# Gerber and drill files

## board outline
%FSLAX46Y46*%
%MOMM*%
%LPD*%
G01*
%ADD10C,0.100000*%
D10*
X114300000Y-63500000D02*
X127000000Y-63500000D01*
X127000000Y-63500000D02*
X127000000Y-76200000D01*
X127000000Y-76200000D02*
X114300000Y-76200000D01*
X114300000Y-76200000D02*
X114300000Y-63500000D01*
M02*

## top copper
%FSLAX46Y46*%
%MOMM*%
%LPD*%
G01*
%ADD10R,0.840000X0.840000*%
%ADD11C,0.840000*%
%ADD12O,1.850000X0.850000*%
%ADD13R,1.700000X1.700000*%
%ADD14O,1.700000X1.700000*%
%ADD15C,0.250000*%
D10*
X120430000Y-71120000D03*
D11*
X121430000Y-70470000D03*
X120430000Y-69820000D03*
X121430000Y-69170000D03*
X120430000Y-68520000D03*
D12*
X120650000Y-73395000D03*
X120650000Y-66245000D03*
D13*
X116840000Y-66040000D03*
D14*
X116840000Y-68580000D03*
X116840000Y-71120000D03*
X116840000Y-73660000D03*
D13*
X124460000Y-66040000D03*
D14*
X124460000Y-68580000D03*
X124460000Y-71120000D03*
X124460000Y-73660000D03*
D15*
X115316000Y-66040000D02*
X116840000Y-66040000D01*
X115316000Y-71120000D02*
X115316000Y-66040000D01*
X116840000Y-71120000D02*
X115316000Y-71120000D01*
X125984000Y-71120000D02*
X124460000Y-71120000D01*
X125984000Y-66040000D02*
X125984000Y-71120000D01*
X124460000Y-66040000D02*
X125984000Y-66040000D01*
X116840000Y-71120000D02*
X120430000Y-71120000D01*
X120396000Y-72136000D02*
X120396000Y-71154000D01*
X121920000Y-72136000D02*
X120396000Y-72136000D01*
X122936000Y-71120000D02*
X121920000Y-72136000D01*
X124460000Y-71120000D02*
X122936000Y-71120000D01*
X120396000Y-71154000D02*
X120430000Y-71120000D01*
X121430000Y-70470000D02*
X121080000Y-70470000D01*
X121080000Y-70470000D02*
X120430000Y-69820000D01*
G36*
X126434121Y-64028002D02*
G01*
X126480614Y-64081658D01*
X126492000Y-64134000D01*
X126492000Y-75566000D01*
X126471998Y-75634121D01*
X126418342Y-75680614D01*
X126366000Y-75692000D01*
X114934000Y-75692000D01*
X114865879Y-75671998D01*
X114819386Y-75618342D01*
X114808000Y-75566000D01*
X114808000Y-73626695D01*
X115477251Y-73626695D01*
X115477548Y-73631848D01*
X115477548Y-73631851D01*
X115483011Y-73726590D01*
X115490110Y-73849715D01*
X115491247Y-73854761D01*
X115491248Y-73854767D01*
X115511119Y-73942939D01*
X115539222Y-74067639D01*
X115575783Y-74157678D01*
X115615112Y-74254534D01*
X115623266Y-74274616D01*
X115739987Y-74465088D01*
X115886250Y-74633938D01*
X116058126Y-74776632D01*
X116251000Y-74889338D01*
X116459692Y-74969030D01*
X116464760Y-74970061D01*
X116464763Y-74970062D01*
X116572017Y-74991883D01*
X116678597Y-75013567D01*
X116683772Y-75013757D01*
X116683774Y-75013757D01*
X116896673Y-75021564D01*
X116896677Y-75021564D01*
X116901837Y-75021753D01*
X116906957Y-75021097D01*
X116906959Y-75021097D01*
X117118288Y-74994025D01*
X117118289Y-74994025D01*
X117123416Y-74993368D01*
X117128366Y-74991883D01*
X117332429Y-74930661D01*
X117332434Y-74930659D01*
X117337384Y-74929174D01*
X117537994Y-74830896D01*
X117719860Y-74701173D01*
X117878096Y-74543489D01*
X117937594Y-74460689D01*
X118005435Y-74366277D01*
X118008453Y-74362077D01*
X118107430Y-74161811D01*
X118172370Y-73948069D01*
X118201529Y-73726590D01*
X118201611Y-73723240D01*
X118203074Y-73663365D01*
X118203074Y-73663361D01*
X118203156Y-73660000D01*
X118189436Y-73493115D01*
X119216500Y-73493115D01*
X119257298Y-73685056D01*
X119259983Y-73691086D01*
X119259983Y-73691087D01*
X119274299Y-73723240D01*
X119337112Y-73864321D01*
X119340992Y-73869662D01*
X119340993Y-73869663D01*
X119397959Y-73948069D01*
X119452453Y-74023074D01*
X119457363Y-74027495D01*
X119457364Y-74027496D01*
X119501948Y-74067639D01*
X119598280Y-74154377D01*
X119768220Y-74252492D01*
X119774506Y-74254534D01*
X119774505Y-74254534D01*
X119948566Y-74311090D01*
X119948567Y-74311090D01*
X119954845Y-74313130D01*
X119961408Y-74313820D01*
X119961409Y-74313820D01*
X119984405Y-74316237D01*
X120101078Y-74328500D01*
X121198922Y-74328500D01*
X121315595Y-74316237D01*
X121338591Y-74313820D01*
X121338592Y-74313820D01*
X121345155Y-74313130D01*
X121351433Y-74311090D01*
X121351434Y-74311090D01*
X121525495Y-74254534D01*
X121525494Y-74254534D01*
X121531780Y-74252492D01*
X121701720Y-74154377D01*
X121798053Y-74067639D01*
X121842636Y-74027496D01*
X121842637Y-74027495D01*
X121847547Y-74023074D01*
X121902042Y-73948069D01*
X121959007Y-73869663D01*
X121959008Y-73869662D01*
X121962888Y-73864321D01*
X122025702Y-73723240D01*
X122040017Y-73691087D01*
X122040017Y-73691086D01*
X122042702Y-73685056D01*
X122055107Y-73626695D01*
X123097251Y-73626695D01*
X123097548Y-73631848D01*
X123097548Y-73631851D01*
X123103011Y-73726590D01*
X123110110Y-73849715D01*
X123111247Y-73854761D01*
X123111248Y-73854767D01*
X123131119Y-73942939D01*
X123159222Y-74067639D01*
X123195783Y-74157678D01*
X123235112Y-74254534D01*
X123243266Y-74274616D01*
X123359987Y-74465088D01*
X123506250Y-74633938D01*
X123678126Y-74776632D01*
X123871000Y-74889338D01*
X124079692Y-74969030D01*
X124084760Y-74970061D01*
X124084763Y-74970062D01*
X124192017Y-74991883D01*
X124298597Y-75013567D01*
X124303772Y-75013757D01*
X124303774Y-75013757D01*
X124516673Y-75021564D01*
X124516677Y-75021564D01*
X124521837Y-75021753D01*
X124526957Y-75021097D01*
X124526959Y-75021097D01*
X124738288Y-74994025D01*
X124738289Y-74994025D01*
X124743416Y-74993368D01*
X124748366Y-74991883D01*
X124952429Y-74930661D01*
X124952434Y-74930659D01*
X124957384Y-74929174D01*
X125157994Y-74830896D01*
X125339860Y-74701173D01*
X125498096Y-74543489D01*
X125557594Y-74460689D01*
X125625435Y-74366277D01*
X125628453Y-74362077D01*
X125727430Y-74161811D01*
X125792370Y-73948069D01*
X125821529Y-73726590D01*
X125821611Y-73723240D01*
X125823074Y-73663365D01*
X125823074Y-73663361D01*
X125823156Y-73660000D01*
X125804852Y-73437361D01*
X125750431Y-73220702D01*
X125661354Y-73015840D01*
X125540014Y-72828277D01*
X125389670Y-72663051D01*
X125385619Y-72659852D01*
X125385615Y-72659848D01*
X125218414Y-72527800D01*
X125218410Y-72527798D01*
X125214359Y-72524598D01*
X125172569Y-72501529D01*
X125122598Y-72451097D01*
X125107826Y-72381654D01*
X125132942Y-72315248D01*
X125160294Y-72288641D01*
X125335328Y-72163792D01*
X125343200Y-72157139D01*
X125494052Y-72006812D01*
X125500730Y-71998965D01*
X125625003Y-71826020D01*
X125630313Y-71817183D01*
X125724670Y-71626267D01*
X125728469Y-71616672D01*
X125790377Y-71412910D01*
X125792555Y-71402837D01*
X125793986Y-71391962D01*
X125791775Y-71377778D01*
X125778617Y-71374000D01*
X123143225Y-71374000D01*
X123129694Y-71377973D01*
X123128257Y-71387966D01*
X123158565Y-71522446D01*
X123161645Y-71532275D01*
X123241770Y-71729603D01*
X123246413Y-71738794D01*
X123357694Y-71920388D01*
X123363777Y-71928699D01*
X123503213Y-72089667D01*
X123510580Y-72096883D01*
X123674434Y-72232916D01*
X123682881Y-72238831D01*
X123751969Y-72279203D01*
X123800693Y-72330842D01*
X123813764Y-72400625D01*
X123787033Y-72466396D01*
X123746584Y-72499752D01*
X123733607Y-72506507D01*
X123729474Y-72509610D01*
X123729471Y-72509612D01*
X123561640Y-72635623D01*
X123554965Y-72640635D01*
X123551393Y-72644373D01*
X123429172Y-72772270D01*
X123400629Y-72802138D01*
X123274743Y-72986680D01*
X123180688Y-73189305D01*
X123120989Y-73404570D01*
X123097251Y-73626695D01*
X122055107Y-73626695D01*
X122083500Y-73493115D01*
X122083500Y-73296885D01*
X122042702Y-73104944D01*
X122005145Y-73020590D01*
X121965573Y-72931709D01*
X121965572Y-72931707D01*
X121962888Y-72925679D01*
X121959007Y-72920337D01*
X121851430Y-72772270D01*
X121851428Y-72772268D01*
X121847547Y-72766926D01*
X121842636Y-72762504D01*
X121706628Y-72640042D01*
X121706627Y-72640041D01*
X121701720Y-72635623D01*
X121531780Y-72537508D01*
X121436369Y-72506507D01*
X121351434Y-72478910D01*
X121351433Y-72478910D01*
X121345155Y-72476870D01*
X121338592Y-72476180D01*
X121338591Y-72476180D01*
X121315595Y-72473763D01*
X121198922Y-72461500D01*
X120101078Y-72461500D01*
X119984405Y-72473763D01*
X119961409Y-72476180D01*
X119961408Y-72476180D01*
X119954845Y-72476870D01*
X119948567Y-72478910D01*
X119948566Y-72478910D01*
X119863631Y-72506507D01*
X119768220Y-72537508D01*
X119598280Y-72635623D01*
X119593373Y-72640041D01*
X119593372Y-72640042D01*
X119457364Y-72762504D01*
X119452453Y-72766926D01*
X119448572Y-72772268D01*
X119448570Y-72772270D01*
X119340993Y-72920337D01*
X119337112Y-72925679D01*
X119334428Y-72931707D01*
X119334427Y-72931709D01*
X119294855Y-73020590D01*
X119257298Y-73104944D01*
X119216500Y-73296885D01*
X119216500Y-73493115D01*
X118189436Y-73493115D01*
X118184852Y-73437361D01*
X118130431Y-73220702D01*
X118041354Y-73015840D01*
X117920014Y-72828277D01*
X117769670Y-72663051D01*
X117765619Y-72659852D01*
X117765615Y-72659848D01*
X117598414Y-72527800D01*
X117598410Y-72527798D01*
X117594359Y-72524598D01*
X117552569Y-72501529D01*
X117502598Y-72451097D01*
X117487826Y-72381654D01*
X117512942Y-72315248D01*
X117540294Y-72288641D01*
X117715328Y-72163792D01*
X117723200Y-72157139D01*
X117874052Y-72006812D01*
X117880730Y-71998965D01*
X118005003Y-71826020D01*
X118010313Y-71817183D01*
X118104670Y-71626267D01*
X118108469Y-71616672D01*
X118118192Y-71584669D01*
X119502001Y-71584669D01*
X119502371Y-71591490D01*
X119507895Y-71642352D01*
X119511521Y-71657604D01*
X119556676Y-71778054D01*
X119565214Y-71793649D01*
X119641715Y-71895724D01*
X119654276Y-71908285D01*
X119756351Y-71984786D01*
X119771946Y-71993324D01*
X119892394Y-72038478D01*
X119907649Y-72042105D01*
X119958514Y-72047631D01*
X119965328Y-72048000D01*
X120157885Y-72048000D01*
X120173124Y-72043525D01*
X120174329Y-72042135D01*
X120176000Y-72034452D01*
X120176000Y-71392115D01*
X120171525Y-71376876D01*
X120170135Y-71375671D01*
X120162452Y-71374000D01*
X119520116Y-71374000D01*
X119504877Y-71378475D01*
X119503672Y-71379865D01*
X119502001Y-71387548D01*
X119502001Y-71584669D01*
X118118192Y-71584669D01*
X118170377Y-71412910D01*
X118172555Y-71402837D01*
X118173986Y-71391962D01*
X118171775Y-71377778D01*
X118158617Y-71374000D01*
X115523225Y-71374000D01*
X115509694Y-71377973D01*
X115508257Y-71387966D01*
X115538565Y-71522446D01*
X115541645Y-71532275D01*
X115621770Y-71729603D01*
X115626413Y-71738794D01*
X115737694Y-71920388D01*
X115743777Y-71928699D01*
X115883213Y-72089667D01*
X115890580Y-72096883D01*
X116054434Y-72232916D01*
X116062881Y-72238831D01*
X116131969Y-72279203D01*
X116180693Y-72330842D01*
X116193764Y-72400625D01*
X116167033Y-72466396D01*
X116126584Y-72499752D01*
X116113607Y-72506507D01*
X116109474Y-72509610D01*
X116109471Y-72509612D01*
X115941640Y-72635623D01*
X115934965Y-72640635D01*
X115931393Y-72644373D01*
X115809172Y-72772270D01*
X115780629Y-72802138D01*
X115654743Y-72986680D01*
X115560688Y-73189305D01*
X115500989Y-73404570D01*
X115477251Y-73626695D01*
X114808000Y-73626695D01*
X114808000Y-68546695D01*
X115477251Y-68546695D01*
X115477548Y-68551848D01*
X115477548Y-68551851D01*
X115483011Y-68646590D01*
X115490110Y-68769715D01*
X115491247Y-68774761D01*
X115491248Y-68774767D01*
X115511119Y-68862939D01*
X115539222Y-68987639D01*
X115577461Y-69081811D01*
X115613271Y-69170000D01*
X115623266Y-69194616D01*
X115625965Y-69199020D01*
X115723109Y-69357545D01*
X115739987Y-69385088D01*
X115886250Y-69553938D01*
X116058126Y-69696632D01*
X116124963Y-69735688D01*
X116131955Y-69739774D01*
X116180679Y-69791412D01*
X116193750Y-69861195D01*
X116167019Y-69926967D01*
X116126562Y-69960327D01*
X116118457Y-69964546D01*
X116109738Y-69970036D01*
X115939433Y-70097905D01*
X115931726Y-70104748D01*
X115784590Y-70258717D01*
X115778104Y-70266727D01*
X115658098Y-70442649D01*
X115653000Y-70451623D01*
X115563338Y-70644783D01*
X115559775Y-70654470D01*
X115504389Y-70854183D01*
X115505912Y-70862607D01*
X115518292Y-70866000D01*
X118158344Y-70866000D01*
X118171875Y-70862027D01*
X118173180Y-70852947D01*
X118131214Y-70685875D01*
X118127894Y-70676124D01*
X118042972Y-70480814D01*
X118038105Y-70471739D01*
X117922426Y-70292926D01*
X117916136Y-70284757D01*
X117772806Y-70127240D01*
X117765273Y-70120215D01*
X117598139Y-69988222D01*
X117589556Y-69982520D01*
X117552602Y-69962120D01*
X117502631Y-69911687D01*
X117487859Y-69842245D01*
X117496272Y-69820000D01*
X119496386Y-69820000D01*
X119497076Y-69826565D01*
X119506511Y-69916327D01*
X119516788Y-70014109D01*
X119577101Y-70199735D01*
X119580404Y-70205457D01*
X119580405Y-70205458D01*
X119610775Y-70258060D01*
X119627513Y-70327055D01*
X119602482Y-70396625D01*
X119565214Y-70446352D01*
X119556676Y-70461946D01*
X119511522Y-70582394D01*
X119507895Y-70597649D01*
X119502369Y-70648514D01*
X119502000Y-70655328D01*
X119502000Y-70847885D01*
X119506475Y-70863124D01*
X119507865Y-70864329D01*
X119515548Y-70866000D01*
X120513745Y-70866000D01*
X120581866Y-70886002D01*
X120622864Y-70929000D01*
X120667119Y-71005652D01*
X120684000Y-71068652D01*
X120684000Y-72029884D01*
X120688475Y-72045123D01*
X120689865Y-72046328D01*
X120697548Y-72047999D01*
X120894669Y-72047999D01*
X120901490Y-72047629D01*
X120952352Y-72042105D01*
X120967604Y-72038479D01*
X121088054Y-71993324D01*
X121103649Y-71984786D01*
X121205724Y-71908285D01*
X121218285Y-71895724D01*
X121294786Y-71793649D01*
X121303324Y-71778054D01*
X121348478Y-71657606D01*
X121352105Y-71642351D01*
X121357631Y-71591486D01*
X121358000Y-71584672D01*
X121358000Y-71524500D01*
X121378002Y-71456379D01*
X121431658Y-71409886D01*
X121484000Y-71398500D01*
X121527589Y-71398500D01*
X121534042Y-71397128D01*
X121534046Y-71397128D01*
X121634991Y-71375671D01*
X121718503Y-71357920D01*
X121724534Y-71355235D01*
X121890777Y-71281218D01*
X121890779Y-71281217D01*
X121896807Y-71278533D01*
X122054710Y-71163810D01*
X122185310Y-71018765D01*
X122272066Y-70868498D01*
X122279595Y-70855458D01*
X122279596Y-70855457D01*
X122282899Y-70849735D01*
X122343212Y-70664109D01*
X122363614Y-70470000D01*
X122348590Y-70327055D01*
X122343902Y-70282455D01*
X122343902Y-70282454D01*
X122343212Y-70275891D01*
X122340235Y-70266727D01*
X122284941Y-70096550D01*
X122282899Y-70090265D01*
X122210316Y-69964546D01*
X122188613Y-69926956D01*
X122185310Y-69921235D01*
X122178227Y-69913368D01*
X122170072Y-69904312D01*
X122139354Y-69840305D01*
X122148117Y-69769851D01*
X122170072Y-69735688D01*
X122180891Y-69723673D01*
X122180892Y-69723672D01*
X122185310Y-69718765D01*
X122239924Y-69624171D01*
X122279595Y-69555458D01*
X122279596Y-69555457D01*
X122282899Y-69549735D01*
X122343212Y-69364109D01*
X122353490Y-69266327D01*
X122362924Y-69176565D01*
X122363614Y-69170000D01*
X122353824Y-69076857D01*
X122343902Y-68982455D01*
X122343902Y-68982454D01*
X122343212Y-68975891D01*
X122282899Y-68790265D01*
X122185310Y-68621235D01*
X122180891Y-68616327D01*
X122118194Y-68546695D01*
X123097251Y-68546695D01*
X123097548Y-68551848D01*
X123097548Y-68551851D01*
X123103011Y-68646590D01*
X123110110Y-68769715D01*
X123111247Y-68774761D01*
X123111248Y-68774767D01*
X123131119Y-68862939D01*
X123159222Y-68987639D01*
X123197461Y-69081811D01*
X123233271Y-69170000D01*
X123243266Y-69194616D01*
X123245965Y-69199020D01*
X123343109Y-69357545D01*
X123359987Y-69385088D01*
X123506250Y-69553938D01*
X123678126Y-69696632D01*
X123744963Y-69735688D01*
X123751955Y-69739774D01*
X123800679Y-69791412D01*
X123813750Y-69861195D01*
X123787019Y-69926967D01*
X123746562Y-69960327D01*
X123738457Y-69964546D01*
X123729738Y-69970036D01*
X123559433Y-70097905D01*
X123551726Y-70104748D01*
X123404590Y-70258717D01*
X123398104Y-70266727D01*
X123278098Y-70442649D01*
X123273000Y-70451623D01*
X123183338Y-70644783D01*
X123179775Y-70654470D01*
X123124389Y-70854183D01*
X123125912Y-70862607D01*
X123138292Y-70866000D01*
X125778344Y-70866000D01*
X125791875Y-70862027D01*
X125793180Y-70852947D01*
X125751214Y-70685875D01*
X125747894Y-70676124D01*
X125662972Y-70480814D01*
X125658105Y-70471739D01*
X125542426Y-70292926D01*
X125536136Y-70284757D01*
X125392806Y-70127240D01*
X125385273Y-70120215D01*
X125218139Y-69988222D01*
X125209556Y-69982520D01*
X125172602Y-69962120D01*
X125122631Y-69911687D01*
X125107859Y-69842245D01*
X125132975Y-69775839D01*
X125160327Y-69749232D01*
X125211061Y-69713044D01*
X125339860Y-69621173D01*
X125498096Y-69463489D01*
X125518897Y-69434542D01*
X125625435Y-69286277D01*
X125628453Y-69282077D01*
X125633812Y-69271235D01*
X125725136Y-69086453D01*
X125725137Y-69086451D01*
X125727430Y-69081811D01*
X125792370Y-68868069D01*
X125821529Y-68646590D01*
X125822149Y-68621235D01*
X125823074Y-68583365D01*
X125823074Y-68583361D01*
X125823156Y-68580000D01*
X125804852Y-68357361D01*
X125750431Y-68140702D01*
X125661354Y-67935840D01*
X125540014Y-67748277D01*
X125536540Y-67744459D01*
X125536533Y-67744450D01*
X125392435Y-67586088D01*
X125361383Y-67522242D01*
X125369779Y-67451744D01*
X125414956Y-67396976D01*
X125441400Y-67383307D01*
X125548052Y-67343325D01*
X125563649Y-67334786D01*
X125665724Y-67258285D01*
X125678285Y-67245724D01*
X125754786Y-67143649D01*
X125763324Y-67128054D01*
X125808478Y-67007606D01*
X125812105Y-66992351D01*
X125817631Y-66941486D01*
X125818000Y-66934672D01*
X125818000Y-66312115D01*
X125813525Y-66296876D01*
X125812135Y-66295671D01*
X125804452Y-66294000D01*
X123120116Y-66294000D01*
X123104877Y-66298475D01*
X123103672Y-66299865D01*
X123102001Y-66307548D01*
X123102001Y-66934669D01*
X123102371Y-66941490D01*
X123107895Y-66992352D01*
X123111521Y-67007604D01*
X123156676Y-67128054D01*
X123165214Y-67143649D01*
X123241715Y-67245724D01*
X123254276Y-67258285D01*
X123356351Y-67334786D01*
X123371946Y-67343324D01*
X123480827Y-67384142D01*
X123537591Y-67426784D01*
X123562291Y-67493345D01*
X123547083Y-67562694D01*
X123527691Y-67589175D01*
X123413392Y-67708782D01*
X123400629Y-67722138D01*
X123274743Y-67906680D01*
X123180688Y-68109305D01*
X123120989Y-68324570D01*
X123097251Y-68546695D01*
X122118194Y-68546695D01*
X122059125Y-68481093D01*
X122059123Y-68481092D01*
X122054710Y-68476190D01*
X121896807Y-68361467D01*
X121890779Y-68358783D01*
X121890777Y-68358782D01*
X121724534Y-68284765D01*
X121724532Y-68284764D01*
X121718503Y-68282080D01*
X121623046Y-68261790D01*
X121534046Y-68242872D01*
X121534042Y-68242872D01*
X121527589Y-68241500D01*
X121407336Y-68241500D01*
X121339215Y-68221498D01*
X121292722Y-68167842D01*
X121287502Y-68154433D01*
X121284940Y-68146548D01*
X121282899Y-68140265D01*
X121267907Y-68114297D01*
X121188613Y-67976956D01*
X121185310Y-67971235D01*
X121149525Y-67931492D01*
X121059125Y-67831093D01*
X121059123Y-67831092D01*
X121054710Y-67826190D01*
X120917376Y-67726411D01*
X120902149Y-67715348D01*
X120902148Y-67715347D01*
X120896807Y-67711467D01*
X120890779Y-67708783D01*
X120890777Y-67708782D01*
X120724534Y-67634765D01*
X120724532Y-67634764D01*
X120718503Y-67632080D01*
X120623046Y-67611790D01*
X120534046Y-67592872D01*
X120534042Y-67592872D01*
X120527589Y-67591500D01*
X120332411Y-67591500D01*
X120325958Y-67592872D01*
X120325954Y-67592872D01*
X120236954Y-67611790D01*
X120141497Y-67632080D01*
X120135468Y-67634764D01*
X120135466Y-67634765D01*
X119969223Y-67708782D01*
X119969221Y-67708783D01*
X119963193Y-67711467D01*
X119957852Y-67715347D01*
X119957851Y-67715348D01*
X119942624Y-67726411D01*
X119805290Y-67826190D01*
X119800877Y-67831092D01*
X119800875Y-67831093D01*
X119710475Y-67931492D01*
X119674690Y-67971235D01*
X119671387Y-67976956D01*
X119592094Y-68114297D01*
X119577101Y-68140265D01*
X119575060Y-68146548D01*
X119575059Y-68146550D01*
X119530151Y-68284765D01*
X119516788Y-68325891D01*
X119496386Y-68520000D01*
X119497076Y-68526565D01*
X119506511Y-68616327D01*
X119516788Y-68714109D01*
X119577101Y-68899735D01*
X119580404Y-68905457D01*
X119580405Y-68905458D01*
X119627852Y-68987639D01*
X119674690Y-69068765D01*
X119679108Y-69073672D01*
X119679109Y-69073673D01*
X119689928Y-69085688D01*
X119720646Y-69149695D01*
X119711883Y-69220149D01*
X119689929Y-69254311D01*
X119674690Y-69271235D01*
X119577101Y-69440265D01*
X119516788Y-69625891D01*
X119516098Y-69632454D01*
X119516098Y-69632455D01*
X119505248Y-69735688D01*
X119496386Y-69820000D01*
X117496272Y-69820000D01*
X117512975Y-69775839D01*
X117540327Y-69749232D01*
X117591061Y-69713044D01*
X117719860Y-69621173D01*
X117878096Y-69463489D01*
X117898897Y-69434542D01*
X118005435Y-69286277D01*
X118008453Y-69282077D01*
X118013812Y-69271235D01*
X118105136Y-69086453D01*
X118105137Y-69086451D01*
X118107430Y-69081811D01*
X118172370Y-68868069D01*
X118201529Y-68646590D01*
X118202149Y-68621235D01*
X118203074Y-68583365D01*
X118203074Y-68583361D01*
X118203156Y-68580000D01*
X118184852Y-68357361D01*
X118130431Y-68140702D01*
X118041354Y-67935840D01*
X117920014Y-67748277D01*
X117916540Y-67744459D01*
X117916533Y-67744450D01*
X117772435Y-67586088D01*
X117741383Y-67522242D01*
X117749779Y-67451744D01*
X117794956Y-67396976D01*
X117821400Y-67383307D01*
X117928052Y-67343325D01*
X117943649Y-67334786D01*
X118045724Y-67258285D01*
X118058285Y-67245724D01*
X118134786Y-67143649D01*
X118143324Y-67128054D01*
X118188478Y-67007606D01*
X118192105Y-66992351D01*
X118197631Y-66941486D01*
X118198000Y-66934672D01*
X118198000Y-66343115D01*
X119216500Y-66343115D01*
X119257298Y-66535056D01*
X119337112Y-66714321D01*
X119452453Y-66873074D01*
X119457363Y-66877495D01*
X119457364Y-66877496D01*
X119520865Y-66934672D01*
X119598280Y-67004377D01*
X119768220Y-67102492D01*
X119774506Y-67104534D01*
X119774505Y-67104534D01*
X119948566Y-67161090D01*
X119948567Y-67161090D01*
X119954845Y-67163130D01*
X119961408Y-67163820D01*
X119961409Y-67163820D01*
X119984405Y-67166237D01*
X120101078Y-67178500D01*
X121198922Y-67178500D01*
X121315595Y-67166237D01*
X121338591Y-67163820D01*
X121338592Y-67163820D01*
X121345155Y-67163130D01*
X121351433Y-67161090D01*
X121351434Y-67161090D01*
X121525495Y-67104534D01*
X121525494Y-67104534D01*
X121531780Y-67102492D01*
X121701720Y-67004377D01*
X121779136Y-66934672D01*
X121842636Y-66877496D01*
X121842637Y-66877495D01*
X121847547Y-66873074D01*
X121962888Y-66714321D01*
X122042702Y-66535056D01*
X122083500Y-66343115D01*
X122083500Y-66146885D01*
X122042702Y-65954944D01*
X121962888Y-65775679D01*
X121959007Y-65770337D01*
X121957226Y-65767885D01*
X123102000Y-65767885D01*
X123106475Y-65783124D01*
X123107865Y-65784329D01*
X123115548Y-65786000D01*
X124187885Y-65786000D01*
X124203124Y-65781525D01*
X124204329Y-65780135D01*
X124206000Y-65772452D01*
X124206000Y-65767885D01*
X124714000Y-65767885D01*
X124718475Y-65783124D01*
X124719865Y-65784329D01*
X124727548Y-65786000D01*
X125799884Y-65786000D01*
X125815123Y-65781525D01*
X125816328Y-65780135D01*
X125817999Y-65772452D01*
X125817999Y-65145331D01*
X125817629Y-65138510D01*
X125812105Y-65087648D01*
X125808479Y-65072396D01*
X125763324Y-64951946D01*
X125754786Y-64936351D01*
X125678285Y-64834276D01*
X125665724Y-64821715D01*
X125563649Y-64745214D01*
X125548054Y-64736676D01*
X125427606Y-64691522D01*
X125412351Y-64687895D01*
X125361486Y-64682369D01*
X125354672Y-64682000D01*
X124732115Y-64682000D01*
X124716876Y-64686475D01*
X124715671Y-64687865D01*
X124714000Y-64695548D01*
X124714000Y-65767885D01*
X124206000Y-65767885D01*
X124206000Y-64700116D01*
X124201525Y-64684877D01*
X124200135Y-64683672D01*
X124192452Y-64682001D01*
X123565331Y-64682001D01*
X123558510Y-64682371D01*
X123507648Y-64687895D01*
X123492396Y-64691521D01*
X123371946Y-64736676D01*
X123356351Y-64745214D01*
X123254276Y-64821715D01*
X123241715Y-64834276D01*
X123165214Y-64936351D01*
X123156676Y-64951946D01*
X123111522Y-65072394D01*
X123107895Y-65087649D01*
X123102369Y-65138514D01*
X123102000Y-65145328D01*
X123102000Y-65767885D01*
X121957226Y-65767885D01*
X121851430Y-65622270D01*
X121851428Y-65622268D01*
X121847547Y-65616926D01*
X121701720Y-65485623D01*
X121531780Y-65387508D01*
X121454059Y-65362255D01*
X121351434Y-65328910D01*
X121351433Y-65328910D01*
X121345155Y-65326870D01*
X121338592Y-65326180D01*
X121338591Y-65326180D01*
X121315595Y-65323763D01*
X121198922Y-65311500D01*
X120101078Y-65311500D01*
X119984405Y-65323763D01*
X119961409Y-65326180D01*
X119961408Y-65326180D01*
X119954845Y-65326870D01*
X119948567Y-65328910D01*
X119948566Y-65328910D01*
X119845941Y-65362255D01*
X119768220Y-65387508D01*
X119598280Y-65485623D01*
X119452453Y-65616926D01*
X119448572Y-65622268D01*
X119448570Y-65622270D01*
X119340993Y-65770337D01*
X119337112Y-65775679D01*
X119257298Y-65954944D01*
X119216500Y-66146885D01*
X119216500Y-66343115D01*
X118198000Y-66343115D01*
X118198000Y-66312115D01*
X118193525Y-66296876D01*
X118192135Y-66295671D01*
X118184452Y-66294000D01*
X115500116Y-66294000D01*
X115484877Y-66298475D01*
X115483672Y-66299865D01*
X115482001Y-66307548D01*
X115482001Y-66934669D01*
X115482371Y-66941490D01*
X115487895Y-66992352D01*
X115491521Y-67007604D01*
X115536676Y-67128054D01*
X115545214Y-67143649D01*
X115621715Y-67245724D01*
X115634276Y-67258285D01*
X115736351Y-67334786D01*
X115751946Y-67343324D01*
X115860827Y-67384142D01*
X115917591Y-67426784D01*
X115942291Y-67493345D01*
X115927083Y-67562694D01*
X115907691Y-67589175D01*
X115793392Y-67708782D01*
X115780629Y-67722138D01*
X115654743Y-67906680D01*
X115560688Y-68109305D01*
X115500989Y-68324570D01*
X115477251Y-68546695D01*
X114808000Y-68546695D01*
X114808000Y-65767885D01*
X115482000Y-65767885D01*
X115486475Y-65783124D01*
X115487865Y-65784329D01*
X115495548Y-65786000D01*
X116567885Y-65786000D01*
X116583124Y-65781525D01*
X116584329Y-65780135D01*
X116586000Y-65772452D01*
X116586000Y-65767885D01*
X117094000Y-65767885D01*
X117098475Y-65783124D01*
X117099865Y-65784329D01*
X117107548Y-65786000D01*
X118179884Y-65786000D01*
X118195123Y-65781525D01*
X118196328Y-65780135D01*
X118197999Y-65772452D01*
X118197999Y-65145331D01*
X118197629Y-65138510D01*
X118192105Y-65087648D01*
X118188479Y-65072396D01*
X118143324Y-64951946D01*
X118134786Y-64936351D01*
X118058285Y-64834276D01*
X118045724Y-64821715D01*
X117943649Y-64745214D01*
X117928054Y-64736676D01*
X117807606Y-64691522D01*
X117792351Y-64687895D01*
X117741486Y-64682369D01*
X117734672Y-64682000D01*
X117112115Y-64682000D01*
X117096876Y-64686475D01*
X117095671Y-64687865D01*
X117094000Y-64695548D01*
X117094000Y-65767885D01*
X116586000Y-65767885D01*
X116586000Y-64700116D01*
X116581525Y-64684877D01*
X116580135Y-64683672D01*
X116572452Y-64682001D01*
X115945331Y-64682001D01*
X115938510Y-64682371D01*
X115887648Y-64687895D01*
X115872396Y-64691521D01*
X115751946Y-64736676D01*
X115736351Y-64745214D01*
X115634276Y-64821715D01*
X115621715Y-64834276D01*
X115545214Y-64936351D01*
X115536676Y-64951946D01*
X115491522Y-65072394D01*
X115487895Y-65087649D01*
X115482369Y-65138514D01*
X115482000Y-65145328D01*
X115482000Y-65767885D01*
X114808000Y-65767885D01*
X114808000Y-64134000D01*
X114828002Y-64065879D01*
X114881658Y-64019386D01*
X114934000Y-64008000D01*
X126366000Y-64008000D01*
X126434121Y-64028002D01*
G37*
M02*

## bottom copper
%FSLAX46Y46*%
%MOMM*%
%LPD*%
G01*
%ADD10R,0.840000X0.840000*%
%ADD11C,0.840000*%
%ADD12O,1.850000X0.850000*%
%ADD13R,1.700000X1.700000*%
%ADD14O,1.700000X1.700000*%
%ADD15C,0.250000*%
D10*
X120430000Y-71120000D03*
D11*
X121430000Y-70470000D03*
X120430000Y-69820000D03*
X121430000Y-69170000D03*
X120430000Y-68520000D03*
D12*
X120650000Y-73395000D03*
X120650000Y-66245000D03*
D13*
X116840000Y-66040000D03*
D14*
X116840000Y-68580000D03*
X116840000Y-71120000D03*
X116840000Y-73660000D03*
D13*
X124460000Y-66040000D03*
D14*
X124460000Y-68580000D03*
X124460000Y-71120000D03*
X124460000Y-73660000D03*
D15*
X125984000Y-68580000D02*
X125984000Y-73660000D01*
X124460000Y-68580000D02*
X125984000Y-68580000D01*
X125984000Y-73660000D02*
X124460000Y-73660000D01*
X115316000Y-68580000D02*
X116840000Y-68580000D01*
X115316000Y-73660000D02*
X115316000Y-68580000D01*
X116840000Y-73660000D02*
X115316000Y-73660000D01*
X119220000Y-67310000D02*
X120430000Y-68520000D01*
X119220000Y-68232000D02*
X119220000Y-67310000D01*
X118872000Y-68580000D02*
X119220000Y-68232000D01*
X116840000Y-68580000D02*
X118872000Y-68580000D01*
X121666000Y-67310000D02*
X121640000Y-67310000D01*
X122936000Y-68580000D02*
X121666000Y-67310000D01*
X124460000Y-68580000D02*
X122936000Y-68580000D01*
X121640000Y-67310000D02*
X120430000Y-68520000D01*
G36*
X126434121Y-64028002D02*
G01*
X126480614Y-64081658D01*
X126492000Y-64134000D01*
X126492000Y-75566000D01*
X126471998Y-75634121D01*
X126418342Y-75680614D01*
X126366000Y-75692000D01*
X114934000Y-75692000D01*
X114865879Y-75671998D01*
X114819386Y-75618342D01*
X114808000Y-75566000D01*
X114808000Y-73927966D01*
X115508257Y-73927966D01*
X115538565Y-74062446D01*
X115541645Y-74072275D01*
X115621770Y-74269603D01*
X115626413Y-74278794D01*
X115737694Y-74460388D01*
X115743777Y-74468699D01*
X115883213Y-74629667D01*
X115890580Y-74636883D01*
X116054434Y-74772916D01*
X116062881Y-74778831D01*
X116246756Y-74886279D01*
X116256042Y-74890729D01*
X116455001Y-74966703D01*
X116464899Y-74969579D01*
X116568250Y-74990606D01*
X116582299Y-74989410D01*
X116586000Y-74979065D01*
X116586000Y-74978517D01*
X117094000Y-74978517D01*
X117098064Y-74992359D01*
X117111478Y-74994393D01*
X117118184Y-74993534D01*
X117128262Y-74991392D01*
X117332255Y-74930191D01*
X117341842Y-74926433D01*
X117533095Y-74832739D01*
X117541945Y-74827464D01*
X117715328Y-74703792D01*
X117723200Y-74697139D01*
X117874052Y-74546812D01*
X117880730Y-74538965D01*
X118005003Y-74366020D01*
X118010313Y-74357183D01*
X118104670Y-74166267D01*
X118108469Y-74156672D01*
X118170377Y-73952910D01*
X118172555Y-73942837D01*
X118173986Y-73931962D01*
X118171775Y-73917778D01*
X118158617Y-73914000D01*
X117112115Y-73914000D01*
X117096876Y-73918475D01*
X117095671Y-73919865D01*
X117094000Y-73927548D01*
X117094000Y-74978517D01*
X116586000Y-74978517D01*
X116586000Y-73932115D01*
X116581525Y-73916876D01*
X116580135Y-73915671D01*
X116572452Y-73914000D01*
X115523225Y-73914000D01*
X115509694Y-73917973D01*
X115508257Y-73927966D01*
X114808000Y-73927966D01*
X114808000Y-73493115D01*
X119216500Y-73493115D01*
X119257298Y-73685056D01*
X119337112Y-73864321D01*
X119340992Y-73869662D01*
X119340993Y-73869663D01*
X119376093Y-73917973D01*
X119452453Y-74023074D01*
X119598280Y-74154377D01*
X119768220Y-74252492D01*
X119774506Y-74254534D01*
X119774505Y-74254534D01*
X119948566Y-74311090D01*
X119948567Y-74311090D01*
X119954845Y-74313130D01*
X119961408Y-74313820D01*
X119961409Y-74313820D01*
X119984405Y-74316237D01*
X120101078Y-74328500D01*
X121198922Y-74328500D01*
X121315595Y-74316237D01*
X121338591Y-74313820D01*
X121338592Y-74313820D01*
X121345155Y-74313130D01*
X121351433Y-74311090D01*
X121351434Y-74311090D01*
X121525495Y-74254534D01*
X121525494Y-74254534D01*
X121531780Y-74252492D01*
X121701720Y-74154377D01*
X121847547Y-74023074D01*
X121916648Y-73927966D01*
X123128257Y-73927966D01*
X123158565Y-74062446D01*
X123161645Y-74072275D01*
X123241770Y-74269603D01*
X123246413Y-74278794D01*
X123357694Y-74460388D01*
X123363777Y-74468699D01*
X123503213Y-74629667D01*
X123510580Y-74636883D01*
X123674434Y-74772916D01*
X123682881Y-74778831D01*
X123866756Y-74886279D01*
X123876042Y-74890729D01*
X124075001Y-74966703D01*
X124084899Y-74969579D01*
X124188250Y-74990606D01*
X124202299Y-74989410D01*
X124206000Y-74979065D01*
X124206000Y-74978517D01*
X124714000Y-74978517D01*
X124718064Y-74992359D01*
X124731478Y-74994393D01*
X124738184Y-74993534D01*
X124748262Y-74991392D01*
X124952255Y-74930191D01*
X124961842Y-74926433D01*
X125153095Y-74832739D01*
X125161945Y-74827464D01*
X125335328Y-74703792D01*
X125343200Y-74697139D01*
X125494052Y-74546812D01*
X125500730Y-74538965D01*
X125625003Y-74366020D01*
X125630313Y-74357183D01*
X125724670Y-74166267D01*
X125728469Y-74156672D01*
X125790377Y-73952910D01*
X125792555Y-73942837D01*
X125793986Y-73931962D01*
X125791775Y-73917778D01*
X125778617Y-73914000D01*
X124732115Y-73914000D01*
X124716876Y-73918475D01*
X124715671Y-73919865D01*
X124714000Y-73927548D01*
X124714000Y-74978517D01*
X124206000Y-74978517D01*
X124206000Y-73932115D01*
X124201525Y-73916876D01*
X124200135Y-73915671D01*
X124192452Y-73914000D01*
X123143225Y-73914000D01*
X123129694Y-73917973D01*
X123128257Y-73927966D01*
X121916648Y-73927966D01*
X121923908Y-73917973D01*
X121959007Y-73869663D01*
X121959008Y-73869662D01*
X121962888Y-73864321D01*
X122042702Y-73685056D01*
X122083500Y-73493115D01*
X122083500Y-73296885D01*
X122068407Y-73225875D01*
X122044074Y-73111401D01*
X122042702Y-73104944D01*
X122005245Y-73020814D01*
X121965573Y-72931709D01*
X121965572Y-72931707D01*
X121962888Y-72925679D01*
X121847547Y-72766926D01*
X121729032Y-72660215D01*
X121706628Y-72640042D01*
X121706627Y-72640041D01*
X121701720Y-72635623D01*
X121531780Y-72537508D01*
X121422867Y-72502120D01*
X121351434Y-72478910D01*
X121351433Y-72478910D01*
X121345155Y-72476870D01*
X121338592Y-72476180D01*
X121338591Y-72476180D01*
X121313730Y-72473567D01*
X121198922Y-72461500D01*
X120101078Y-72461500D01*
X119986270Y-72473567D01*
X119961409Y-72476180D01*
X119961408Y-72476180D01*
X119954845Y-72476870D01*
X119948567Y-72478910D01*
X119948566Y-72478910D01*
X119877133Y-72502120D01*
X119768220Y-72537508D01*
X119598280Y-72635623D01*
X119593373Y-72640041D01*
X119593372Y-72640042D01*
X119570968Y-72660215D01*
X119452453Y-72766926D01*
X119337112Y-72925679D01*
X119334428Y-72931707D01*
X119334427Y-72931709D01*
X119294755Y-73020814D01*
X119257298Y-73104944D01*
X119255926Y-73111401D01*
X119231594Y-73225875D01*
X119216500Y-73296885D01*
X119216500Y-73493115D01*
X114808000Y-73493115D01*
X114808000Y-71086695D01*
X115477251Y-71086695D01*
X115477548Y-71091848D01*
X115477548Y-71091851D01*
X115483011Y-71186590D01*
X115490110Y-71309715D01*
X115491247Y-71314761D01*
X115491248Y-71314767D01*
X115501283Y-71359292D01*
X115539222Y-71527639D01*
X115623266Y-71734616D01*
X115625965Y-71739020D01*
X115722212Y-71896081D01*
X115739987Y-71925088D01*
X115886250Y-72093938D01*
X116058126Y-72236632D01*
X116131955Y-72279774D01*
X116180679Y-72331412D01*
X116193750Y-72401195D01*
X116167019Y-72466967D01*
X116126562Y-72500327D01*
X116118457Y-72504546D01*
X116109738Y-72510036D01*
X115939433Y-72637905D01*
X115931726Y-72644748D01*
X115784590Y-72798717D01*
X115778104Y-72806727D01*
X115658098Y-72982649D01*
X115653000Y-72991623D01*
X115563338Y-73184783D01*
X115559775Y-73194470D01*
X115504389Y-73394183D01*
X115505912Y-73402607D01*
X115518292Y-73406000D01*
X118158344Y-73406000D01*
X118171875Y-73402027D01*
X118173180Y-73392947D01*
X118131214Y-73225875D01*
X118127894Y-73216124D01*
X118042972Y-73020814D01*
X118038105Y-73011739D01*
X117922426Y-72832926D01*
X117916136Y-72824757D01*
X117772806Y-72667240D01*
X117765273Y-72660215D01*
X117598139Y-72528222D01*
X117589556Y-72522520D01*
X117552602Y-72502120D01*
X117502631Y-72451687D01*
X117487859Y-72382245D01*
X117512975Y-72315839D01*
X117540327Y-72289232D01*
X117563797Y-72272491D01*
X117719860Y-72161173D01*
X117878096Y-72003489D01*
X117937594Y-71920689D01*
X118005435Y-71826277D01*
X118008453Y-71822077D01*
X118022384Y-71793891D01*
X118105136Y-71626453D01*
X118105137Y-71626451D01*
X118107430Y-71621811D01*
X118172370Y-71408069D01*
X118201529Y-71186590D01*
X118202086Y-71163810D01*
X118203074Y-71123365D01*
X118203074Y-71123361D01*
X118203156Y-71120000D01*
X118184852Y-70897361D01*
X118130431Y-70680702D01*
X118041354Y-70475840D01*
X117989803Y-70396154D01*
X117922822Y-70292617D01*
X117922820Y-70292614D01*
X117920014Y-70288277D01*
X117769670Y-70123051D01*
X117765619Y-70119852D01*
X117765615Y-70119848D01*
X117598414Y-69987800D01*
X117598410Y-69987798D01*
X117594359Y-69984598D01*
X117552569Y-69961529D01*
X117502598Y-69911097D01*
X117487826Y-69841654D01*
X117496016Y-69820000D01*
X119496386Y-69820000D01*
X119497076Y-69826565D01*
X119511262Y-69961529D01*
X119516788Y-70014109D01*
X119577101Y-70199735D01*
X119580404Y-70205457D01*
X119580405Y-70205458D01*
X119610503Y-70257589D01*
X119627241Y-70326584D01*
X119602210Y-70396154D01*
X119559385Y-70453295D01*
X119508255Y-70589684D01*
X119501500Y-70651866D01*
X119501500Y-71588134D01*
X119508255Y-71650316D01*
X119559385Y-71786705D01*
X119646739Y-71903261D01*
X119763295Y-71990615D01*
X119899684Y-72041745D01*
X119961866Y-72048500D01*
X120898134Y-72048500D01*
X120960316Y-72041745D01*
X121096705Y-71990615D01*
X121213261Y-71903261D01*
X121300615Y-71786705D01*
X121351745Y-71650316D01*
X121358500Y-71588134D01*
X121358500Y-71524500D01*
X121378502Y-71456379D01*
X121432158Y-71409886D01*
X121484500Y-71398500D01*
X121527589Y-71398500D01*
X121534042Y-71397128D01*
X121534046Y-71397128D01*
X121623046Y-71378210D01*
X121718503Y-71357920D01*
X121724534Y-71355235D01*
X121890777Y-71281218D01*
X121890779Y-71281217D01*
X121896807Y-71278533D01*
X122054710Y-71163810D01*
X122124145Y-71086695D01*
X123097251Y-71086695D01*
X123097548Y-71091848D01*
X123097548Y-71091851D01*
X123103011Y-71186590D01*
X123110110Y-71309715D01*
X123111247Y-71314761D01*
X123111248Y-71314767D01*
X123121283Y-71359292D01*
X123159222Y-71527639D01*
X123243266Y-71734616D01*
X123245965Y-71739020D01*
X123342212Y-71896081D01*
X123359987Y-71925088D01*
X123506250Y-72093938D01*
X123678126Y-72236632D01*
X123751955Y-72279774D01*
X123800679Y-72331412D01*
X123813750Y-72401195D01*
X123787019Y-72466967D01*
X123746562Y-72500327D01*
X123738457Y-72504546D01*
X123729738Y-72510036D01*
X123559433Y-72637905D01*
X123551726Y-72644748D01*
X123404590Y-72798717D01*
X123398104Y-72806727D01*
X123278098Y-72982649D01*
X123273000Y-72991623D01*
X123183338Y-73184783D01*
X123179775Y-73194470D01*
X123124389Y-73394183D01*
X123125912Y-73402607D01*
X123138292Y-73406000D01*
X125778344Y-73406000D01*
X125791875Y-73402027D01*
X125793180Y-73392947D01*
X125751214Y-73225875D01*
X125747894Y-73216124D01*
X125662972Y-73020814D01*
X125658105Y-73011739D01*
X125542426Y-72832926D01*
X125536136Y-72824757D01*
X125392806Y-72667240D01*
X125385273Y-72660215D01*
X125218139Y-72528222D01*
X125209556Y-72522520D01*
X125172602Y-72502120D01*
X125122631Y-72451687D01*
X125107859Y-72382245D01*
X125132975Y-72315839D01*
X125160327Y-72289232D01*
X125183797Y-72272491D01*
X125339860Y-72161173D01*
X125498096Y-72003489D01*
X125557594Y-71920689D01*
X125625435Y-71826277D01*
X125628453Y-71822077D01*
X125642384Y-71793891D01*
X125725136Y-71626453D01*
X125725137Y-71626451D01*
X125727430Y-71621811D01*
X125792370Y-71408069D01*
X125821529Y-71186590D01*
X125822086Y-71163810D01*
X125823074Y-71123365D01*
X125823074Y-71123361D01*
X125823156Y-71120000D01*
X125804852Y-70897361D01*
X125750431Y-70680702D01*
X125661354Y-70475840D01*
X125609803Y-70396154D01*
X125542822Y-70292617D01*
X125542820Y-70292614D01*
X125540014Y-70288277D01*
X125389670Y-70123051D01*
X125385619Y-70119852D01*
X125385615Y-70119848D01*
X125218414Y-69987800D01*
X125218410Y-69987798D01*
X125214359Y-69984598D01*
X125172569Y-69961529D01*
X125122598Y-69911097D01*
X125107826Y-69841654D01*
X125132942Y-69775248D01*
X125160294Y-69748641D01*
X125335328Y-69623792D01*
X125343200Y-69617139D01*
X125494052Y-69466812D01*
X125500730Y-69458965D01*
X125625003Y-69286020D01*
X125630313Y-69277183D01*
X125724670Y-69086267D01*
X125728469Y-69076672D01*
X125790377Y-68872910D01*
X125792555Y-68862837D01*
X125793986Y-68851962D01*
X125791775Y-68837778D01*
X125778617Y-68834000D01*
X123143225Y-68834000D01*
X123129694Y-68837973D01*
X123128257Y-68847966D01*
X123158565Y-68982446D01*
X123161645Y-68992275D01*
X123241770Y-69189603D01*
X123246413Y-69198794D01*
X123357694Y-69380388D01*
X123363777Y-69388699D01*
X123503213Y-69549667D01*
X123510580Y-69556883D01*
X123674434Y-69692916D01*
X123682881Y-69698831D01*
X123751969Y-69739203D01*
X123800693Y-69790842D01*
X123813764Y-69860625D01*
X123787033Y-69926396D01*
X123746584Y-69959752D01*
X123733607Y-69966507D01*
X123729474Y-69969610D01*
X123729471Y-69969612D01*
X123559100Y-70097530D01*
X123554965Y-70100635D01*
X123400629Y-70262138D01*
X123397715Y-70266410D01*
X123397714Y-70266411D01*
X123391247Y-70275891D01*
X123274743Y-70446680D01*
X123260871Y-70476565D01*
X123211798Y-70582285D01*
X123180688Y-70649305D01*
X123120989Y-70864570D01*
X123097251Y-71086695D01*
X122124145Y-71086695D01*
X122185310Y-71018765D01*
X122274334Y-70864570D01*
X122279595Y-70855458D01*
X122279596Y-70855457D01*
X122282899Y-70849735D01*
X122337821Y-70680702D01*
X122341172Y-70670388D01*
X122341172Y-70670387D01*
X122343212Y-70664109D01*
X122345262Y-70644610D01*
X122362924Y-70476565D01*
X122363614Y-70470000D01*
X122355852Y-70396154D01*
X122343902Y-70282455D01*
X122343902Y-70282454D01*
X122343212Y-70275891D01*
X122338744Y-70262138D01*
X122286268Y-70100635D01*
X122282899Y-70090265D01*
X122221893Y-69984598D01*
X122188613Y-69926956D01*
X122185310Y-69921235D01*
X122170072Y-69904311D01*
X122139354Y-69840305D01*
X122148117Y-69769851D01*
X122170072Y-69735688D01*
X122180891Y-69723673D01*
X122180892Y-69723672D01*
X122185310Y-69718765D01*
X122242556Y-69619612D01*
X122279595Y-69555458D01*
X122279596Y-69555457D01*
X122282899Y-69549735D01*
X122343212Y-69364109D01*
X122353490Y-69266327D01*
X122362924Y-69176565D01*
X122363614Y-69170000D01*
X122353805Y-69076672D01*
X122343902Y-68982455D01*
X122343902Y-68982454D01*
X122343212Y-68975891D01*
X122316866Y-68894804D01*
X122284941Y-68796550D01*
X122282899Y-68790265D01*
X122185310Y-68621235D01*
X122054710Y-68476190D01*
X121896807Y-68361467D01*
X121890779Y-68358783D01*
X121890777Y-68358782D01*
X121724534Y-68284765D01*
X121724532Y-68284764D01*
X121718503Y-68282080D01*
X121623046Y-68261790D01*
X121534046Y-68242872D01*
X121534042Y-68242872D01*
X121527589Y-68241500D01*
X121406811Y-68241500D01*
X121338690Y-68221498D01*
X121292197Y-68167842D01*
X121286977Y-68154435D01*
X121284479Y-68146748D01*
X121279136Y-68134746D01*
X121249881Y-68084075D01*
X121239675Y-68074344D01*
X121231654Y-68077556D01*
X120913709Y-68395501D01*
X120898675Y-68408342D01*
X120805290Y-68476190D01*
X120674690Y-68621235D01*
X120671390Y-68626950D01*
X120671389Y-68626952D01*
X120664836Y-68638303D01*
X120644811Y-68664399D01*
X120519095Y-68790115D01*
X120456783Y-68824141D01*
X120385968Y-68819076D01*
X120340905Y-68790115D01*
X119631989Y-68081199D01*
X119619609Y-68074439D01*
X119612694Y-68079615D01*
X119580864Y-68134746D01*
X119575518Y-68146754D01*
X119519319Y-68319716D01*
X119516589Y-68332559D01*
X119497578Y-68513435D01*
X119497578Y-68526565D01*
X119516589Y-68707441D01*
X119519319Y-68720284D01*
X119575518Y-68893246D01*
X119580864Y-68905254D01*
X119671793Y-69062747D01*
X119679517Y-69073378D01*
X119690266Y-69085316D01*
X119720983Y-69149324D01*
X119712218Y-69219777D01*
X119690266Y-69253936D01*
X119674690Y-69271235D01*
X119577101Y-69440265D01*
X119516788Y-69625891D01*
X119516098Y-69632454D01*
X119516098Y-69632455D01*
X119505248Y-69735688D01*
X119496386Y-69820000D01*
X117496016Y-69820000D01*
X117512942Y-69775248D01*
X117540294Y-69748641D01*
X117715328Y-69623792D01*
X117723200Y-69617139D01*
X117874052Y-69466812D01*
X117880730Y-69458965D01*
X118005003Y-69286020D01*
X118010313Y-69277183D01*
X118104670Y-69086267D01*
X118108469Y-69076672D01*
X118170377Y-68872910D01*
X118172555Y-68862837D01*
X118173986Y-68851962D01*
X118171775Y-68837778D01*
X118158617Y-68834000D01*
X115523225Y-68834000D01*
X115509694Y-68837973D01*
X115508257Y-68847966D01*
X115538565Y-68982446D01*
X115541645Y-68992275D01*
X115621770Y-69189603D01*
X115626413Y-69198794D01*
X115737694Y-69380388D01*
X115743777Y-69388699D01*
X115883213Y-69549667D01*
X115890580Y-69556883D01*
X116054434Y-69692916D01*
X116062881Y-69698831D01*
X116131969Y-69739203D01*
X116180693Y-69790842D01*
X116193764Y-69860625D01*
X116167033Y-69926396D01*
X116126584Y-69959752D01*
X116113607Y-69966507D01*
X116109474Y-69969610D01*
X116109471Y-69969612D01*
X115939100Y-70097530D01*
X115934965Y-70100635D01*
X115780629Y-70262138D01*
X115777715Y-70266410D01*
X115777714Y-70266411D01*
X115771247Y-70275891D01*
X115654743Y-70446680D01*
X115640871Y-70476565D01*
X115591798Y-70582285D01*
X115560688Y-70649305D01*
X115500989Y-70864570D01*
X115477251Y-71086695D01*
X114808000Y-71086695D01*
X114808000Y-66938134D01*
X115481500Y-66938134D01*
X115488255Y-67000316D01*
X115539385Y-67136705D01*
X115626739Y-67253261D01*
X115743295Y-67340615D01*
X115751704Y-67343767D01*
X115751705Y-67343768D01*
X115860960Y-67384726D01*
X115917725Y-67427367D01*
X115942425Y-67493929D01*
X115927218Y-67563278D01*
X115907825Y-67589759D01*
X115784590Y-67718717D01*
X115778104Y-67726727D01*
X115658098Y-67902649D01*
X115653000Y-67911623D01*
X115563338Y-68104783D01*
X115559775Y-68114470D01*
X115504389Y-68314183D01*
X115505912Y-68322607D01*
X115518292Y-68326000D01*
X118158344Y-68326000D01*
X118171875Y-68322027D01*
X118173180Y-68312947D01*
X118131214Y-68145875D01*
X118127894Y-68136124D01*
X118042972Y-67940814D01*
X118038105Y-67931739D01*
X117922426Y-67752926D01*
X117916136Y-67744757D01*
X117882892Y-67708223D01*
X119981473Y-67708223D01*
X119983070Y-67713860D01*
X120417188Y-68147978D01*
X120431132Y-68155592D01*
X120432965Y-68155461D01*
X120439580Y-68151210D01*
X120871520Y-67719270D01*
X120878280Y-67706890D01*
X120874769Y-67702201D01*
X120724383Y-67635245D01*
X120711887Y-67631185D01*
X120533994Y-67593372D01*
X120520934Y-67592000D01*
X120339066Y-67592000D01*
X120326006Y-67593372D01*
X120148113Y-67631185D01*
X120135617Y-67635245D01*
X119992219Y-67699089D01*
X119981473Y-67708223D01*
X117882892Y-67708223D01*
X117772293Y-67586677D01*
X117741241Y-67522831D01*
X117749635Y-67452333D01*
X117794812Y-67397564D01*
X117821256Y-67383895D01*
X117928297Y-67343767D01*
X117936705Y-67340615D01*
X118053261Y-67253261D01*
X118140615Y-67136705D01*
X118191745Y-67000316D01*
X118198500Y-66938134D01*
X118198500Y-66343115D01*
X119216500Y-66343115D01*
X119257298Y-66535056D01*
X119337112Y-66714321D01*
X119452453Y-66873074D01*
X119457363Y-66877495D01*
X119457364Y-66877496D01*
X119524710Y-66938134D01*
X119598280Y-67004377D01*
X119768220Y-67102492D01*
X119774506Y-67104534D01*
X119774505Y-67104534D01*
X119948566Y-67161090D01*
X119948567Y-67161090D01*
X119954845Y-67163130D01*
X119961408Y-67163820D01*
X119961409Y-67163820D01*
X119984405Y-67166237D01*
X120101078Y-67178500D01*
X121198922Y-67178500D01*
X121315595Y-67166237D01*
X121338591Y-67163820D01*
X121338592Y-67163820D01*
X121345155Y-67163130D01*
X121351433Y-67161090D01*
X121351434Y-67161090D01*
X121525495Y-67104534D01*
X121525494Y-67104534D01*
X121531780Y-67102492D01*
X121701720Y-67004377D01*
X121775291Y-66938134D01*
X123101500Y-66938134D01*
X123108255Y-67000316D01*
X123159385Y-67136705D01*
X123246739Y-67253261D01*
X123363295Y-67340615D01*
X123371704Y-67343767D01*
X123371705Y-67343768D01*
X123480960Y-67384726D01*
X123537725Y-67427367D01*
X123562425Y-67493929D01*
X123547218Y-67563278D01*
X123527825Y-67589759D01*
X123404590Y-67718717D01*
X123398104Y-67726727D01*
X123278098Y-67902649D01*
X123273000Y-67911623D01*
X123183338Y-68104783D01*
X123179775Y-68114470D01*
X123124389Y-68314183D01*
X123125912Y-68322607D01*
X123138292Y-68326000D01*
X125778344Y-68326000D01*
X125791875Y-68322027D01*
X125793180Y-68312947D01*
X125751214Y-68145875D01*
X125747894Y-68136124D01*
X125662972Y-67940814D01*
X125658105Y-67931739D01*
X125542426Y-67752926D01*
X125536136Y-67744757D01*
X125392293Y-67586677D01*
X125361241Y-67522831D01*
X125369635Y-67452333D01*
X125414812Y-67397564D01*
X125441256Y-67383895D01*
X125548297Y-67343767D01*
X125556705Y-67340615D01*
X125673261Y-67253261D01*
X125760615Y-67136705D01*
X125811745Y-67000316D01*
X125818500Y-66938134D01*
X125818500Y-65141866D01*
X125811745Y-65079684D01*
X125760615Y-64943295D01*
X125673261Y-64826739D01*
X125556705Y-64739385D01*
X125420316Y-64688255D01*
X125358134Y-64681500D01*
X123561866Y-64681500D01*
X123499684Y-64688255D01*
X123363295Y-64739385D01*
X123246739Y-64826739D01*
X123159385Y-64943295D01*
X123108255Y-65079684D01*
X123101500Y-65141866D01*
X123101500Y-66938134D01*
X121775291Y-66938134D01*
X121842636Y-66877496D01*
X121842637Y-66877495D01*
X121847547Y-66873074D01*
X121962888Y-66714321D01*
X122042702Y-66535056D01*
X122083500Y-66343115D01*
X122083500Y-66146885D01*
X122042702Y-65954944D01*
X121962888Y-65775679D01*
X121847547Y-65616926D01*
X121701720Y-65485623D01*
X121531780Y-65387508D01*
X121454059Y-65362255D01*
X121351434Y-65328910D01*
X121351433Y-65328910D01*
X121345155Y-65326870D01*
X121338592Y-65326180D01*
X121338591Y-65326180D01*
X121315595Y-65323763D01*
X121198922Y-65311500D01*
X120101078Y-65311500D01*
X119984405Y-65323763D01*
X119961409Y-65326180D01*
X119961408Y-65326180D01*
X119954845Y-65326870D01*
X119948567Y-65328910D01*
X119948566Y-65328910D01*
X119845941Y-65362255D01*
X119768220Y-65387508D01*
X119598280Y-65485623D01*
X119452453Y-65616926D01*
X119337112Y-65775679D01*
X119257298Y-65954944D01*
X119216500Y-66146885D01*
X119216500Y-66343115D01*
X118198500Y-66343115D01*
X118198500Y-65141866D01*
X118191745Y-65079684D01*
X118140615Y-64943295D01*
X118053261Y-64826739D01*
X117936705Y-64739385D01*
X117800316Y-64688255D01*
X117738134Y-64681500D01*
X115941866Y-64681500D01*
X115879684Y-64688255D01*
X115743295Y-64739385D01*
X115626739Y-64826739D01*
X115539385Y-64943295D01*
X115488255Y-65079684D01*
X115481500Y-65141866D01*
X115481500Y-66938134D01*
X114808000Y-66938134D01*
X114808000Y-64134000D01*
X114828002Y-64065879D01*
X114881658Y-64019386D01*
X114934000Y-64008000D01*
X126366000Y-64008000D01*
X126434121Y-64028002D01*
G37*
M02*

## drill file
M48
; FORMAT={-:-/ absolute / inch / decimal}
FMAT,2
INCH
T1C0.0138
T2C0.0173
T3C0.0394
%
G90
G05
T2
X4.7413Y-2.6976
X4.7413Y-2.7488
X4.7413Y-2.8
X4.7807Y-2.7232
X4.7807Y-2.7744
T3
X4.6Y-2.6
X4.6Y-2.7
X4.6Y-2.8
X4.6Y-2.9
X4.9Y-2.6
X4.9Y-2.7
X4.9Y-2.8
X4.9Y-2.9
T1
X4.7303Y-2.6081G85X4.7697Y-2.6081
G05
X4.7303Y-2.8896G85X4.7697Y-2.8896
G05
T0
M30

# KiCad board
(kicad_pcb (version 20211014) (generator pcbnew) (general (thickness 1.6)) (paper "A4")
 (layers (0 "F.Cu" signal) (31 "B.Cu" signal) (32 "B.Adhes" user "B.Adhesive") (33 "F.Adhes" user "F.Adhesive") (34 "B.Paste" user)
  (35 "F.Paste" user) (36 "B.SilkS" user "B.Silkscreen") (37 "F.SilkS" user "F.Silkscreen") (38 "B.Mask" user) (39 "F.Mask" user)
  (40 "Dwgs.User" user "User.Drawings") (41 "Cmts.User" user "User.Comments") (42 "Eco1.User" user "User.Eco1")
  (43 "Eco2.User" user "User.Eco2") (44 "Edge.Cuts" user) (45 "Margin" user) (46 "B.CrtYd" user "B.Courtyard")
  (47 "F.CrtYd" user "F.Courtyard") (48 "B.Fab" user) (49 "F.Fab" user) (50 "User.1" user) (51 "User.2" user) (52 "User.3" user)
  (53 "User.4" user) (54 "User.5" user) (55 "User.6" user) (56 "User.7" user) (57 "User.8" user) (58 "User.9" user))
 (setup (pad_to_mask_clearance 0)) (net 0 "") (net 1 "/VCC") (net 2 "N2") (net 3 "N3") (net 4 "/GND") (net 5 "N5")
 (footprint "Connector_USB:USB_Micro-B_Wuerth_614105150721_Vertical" (layer "F.Cu") (at 120.43 71.12 90)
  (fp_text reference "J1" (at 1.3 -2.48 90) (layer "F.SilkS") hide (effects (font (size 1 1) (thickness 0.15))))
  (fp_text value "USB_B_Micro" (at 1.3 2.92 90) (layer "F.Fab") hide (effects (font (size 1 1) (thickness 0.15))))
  (pad "1" thru_hole rect (at 0 0 90) (size 0.84 0.84) (drill 0.44) (layers *.Cu *.Mask) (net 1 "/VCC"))
  (pad "2" thru_hole circle (at 0.65 1 90) (size 0.84 0.84) (drill 0.44) (layers *.Cu *.Mask) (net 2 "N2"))
  (pad "3" thru_hole circle (at 1.3 0 90) (size 0.84 0.84) (drill 0.44) (layers *.Cu *.Mask) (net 2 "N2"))
  (pad "4" thru_hole circle (at 1.95 1 90) (size 0.84 0.84) (drill 0.44) (layers *.Cu *.Mask) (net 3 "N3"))
  (pad "5" thru_hole circle (at 2.6 0 90) (size 0.84 0.84) (drill 0.44) (layers *.Cu *.Mask) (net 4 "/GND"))
  (pad "6" thru_hole oval (at -2.275 0.22 90) (size 0.85 1.85) (drill oval 0.35 1.35) (layers *.Cu *.Mask) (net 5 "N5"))
  (pad "6" thru_hole oval (at 4.875 0.22 90) (size 0.85 1.85) (drill oval 0.35 1.35) (layers *.Cu *.Mask) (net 5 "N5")))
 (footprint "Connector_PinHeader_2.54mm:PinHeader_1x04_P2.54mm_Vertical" (layer "B.Cu") (at 116.84 66.04 180)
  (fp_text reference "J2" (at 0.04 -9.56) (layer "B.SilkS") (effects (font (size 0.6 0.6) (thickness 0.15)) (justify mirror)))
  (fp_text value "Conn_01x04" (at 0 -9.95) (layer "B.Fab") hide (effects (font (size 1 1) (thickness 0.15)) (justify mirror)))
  (pad "1" thru_hole rect (at 0 0 180) (size 1.7 1.7) (drill 1) (layers *.Cu *.Mask) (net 1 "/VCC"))
  (pad "2" thru_hole oval (at 0 -2.54 180) (size 1.7 1.7) (drill 1) (layers *.Cu *.Mask) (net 4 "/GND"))
  (pad "3" thru_hole oval (at 0 -5.08 180) (size 1.7 1.7) (drill 1) (layers *.Cu *.Mask) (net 1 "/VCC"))
  (pad "4" thru_hole oval (at 0 -7.62 180) (size 1.7 1.7) (drill 1) (layers *.Cu *.Mask) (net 4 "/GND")))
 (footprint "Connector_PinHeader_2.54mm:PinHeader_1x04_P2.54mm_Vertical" (layer "B.Cu") (at 124.46 66.04 180)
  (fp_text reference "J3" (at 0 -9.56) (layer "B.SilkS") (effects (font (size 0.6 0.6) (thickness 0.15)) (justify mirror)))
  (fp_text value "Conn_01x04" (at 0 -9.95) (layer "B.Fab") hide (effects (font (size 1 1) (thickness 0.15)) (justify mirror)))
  (pad "1" thru_hole rect (at 0 0 180) (size 1.7 1.7) (drill 1) (layers *.Cu *.Mask) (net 1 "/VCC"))
  (pad "2" thru_hole oval (at 0 -2.54 180) (size 1.7 1.7) (drill 1) (layers *.Cu *.Mask) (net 4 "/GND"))
  (pad "3" thru_hole oval (at 0 -5.08 180) (size 1.7 1.7) (drill 1) (layers *.Cu *.Mask) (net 1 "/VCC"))
  (pad "4" thru_hole oval (at 0 -7.62 180) (size 1.7 1.7) (drill 1) (layers *.Cu *.Mask) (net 4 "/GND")))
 (gr_rect (start 114.3 63.5) (end 127 76.2) (layer "Edge.Cuts") (width 0.1) (fill none))
 (segment (start 121.43 70.47) (end 121.08 70.47) (width 0.25) (layer "F.Cu") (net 2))
 (segment (start 121.08 70.47) (end 120.43 69.82) (width 0.25) (layer "F.Cu") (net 2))
 (segment (start 124.46 71.12) (end 122.936 71.12) (width 0.25) (layer "F.Cu") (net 1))
 (segment (start 115.316 66.04) (end 116.84 66.04) (width 0.25) (layer "F.Cu") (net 1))
 (segment (start 124.46 66.04) (end 125.984 66.04) (width 0.25) (layer "F.Cu") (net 1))
 (segment (start 115.316 71.12) (end 115.316 66.04) (width 0.25) (layer "F.Cu") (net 1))
 (segment (start 120.396 72.136) (end 120.396 71.154) (width 0.25) (layer "F.Cu") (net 1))
 (segment (start 121.92 72.136) (end 120.396 72.136) (width 0.25) (layer "F.Cu") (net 1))
 (segment (start 125.984 71.12) (end 124.46 71.12) (width 0.25) (layer "F.Cu") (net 1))
 (segment (start 120.396 71.154) (end 120.43 71.12) (width 0.25) (layer "F.Cu") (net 1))
 (segment (start 125.984 66.04) (end 125.984 71.12) (width 0.25) (layer "F.Cu") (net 1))
 (segment (start 116.84 71.12) (end 115.316 71.12) (width 0.25) (layer "F.Cu") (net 1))
 (segment (start 116.84 71.12) (end 120.43 71.12) (width 0.25) (layer "F.Cu") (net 1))
 (segment (start 122.936 71.12) (end 121.92 72.136) (width 0.25) (layer "F.Cu") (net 1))
 (segment (start 116.84 68.58) (end 118.872 68.58) (width 0.25) (layer "B.Cu") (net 4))
 (segment (start 124.46 68.58) (end 125.984 68.58) (width 0.25) (layer "B.Cu") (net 4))
 (segment (start 118.872 68.58) (end 119.22 68.232) (width 0.25) (layer "B.Cu") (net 4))
 (segment (start 119.22 67.31) (end 120.43 68.52) (width 0.25) (layer "B.Cu") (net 4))
 (segment (start 121.666 67.31) (end 121.64 67.31) (width 0.25) (layer "B.Cu") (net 4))
 (segment (start 125.984 73.66) (end 124.46 73.66) (width 0.25) (layer "B.Cu") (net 4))
 (segment (start 115.316 68.58) (end 116.84 68.58) (width 0.25) (layer "B.Cu") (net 4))
 (segment (start 116.84 73.66) (end 115.316 73.66) (width 0.25) (layer "B.Cu") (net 4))
 (segment (start 121.64 67.31) (end 120.43 68.52) (width 0.25) (layer "B.Cu") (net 4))
 (segment (start 115.316 73.66) (end 115.316 68.58) (width 0.25) (layer "B.Cu") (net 4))
 (segment (start 119.22 68.232) (end 119.22 67.31) (width 0.25) (layer "B.Cu") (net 4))
 (segment (start 122.936 68.58) (end 121.666 67.31) (width 0.25) (layer "B.Cu") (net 4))
 (segment (start 124.46 68.58) (end 122.936 68.58) (width 0.25) (layer "B.Cu") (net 4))
 (segment (start 125.984 68.58) (end 125.984 73.66) (width 0.25) (layer "B.Cu") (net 4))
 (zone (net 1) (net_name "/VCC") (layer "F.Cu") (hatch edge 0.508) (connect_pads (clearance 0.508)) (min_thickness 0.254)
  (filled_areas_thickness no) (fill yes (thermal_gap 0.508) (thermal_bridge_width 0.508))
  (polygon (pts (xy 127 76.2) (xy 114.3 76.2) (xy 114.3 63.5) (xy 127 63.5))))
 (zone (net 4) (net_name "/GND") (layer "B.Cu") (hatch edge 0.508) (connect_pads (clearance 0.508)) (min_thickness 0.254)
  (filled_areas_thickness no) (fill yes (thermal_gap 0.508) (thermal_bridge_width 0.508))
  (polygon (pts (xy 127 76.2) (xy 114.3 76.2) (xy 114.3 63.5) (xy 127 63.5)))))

